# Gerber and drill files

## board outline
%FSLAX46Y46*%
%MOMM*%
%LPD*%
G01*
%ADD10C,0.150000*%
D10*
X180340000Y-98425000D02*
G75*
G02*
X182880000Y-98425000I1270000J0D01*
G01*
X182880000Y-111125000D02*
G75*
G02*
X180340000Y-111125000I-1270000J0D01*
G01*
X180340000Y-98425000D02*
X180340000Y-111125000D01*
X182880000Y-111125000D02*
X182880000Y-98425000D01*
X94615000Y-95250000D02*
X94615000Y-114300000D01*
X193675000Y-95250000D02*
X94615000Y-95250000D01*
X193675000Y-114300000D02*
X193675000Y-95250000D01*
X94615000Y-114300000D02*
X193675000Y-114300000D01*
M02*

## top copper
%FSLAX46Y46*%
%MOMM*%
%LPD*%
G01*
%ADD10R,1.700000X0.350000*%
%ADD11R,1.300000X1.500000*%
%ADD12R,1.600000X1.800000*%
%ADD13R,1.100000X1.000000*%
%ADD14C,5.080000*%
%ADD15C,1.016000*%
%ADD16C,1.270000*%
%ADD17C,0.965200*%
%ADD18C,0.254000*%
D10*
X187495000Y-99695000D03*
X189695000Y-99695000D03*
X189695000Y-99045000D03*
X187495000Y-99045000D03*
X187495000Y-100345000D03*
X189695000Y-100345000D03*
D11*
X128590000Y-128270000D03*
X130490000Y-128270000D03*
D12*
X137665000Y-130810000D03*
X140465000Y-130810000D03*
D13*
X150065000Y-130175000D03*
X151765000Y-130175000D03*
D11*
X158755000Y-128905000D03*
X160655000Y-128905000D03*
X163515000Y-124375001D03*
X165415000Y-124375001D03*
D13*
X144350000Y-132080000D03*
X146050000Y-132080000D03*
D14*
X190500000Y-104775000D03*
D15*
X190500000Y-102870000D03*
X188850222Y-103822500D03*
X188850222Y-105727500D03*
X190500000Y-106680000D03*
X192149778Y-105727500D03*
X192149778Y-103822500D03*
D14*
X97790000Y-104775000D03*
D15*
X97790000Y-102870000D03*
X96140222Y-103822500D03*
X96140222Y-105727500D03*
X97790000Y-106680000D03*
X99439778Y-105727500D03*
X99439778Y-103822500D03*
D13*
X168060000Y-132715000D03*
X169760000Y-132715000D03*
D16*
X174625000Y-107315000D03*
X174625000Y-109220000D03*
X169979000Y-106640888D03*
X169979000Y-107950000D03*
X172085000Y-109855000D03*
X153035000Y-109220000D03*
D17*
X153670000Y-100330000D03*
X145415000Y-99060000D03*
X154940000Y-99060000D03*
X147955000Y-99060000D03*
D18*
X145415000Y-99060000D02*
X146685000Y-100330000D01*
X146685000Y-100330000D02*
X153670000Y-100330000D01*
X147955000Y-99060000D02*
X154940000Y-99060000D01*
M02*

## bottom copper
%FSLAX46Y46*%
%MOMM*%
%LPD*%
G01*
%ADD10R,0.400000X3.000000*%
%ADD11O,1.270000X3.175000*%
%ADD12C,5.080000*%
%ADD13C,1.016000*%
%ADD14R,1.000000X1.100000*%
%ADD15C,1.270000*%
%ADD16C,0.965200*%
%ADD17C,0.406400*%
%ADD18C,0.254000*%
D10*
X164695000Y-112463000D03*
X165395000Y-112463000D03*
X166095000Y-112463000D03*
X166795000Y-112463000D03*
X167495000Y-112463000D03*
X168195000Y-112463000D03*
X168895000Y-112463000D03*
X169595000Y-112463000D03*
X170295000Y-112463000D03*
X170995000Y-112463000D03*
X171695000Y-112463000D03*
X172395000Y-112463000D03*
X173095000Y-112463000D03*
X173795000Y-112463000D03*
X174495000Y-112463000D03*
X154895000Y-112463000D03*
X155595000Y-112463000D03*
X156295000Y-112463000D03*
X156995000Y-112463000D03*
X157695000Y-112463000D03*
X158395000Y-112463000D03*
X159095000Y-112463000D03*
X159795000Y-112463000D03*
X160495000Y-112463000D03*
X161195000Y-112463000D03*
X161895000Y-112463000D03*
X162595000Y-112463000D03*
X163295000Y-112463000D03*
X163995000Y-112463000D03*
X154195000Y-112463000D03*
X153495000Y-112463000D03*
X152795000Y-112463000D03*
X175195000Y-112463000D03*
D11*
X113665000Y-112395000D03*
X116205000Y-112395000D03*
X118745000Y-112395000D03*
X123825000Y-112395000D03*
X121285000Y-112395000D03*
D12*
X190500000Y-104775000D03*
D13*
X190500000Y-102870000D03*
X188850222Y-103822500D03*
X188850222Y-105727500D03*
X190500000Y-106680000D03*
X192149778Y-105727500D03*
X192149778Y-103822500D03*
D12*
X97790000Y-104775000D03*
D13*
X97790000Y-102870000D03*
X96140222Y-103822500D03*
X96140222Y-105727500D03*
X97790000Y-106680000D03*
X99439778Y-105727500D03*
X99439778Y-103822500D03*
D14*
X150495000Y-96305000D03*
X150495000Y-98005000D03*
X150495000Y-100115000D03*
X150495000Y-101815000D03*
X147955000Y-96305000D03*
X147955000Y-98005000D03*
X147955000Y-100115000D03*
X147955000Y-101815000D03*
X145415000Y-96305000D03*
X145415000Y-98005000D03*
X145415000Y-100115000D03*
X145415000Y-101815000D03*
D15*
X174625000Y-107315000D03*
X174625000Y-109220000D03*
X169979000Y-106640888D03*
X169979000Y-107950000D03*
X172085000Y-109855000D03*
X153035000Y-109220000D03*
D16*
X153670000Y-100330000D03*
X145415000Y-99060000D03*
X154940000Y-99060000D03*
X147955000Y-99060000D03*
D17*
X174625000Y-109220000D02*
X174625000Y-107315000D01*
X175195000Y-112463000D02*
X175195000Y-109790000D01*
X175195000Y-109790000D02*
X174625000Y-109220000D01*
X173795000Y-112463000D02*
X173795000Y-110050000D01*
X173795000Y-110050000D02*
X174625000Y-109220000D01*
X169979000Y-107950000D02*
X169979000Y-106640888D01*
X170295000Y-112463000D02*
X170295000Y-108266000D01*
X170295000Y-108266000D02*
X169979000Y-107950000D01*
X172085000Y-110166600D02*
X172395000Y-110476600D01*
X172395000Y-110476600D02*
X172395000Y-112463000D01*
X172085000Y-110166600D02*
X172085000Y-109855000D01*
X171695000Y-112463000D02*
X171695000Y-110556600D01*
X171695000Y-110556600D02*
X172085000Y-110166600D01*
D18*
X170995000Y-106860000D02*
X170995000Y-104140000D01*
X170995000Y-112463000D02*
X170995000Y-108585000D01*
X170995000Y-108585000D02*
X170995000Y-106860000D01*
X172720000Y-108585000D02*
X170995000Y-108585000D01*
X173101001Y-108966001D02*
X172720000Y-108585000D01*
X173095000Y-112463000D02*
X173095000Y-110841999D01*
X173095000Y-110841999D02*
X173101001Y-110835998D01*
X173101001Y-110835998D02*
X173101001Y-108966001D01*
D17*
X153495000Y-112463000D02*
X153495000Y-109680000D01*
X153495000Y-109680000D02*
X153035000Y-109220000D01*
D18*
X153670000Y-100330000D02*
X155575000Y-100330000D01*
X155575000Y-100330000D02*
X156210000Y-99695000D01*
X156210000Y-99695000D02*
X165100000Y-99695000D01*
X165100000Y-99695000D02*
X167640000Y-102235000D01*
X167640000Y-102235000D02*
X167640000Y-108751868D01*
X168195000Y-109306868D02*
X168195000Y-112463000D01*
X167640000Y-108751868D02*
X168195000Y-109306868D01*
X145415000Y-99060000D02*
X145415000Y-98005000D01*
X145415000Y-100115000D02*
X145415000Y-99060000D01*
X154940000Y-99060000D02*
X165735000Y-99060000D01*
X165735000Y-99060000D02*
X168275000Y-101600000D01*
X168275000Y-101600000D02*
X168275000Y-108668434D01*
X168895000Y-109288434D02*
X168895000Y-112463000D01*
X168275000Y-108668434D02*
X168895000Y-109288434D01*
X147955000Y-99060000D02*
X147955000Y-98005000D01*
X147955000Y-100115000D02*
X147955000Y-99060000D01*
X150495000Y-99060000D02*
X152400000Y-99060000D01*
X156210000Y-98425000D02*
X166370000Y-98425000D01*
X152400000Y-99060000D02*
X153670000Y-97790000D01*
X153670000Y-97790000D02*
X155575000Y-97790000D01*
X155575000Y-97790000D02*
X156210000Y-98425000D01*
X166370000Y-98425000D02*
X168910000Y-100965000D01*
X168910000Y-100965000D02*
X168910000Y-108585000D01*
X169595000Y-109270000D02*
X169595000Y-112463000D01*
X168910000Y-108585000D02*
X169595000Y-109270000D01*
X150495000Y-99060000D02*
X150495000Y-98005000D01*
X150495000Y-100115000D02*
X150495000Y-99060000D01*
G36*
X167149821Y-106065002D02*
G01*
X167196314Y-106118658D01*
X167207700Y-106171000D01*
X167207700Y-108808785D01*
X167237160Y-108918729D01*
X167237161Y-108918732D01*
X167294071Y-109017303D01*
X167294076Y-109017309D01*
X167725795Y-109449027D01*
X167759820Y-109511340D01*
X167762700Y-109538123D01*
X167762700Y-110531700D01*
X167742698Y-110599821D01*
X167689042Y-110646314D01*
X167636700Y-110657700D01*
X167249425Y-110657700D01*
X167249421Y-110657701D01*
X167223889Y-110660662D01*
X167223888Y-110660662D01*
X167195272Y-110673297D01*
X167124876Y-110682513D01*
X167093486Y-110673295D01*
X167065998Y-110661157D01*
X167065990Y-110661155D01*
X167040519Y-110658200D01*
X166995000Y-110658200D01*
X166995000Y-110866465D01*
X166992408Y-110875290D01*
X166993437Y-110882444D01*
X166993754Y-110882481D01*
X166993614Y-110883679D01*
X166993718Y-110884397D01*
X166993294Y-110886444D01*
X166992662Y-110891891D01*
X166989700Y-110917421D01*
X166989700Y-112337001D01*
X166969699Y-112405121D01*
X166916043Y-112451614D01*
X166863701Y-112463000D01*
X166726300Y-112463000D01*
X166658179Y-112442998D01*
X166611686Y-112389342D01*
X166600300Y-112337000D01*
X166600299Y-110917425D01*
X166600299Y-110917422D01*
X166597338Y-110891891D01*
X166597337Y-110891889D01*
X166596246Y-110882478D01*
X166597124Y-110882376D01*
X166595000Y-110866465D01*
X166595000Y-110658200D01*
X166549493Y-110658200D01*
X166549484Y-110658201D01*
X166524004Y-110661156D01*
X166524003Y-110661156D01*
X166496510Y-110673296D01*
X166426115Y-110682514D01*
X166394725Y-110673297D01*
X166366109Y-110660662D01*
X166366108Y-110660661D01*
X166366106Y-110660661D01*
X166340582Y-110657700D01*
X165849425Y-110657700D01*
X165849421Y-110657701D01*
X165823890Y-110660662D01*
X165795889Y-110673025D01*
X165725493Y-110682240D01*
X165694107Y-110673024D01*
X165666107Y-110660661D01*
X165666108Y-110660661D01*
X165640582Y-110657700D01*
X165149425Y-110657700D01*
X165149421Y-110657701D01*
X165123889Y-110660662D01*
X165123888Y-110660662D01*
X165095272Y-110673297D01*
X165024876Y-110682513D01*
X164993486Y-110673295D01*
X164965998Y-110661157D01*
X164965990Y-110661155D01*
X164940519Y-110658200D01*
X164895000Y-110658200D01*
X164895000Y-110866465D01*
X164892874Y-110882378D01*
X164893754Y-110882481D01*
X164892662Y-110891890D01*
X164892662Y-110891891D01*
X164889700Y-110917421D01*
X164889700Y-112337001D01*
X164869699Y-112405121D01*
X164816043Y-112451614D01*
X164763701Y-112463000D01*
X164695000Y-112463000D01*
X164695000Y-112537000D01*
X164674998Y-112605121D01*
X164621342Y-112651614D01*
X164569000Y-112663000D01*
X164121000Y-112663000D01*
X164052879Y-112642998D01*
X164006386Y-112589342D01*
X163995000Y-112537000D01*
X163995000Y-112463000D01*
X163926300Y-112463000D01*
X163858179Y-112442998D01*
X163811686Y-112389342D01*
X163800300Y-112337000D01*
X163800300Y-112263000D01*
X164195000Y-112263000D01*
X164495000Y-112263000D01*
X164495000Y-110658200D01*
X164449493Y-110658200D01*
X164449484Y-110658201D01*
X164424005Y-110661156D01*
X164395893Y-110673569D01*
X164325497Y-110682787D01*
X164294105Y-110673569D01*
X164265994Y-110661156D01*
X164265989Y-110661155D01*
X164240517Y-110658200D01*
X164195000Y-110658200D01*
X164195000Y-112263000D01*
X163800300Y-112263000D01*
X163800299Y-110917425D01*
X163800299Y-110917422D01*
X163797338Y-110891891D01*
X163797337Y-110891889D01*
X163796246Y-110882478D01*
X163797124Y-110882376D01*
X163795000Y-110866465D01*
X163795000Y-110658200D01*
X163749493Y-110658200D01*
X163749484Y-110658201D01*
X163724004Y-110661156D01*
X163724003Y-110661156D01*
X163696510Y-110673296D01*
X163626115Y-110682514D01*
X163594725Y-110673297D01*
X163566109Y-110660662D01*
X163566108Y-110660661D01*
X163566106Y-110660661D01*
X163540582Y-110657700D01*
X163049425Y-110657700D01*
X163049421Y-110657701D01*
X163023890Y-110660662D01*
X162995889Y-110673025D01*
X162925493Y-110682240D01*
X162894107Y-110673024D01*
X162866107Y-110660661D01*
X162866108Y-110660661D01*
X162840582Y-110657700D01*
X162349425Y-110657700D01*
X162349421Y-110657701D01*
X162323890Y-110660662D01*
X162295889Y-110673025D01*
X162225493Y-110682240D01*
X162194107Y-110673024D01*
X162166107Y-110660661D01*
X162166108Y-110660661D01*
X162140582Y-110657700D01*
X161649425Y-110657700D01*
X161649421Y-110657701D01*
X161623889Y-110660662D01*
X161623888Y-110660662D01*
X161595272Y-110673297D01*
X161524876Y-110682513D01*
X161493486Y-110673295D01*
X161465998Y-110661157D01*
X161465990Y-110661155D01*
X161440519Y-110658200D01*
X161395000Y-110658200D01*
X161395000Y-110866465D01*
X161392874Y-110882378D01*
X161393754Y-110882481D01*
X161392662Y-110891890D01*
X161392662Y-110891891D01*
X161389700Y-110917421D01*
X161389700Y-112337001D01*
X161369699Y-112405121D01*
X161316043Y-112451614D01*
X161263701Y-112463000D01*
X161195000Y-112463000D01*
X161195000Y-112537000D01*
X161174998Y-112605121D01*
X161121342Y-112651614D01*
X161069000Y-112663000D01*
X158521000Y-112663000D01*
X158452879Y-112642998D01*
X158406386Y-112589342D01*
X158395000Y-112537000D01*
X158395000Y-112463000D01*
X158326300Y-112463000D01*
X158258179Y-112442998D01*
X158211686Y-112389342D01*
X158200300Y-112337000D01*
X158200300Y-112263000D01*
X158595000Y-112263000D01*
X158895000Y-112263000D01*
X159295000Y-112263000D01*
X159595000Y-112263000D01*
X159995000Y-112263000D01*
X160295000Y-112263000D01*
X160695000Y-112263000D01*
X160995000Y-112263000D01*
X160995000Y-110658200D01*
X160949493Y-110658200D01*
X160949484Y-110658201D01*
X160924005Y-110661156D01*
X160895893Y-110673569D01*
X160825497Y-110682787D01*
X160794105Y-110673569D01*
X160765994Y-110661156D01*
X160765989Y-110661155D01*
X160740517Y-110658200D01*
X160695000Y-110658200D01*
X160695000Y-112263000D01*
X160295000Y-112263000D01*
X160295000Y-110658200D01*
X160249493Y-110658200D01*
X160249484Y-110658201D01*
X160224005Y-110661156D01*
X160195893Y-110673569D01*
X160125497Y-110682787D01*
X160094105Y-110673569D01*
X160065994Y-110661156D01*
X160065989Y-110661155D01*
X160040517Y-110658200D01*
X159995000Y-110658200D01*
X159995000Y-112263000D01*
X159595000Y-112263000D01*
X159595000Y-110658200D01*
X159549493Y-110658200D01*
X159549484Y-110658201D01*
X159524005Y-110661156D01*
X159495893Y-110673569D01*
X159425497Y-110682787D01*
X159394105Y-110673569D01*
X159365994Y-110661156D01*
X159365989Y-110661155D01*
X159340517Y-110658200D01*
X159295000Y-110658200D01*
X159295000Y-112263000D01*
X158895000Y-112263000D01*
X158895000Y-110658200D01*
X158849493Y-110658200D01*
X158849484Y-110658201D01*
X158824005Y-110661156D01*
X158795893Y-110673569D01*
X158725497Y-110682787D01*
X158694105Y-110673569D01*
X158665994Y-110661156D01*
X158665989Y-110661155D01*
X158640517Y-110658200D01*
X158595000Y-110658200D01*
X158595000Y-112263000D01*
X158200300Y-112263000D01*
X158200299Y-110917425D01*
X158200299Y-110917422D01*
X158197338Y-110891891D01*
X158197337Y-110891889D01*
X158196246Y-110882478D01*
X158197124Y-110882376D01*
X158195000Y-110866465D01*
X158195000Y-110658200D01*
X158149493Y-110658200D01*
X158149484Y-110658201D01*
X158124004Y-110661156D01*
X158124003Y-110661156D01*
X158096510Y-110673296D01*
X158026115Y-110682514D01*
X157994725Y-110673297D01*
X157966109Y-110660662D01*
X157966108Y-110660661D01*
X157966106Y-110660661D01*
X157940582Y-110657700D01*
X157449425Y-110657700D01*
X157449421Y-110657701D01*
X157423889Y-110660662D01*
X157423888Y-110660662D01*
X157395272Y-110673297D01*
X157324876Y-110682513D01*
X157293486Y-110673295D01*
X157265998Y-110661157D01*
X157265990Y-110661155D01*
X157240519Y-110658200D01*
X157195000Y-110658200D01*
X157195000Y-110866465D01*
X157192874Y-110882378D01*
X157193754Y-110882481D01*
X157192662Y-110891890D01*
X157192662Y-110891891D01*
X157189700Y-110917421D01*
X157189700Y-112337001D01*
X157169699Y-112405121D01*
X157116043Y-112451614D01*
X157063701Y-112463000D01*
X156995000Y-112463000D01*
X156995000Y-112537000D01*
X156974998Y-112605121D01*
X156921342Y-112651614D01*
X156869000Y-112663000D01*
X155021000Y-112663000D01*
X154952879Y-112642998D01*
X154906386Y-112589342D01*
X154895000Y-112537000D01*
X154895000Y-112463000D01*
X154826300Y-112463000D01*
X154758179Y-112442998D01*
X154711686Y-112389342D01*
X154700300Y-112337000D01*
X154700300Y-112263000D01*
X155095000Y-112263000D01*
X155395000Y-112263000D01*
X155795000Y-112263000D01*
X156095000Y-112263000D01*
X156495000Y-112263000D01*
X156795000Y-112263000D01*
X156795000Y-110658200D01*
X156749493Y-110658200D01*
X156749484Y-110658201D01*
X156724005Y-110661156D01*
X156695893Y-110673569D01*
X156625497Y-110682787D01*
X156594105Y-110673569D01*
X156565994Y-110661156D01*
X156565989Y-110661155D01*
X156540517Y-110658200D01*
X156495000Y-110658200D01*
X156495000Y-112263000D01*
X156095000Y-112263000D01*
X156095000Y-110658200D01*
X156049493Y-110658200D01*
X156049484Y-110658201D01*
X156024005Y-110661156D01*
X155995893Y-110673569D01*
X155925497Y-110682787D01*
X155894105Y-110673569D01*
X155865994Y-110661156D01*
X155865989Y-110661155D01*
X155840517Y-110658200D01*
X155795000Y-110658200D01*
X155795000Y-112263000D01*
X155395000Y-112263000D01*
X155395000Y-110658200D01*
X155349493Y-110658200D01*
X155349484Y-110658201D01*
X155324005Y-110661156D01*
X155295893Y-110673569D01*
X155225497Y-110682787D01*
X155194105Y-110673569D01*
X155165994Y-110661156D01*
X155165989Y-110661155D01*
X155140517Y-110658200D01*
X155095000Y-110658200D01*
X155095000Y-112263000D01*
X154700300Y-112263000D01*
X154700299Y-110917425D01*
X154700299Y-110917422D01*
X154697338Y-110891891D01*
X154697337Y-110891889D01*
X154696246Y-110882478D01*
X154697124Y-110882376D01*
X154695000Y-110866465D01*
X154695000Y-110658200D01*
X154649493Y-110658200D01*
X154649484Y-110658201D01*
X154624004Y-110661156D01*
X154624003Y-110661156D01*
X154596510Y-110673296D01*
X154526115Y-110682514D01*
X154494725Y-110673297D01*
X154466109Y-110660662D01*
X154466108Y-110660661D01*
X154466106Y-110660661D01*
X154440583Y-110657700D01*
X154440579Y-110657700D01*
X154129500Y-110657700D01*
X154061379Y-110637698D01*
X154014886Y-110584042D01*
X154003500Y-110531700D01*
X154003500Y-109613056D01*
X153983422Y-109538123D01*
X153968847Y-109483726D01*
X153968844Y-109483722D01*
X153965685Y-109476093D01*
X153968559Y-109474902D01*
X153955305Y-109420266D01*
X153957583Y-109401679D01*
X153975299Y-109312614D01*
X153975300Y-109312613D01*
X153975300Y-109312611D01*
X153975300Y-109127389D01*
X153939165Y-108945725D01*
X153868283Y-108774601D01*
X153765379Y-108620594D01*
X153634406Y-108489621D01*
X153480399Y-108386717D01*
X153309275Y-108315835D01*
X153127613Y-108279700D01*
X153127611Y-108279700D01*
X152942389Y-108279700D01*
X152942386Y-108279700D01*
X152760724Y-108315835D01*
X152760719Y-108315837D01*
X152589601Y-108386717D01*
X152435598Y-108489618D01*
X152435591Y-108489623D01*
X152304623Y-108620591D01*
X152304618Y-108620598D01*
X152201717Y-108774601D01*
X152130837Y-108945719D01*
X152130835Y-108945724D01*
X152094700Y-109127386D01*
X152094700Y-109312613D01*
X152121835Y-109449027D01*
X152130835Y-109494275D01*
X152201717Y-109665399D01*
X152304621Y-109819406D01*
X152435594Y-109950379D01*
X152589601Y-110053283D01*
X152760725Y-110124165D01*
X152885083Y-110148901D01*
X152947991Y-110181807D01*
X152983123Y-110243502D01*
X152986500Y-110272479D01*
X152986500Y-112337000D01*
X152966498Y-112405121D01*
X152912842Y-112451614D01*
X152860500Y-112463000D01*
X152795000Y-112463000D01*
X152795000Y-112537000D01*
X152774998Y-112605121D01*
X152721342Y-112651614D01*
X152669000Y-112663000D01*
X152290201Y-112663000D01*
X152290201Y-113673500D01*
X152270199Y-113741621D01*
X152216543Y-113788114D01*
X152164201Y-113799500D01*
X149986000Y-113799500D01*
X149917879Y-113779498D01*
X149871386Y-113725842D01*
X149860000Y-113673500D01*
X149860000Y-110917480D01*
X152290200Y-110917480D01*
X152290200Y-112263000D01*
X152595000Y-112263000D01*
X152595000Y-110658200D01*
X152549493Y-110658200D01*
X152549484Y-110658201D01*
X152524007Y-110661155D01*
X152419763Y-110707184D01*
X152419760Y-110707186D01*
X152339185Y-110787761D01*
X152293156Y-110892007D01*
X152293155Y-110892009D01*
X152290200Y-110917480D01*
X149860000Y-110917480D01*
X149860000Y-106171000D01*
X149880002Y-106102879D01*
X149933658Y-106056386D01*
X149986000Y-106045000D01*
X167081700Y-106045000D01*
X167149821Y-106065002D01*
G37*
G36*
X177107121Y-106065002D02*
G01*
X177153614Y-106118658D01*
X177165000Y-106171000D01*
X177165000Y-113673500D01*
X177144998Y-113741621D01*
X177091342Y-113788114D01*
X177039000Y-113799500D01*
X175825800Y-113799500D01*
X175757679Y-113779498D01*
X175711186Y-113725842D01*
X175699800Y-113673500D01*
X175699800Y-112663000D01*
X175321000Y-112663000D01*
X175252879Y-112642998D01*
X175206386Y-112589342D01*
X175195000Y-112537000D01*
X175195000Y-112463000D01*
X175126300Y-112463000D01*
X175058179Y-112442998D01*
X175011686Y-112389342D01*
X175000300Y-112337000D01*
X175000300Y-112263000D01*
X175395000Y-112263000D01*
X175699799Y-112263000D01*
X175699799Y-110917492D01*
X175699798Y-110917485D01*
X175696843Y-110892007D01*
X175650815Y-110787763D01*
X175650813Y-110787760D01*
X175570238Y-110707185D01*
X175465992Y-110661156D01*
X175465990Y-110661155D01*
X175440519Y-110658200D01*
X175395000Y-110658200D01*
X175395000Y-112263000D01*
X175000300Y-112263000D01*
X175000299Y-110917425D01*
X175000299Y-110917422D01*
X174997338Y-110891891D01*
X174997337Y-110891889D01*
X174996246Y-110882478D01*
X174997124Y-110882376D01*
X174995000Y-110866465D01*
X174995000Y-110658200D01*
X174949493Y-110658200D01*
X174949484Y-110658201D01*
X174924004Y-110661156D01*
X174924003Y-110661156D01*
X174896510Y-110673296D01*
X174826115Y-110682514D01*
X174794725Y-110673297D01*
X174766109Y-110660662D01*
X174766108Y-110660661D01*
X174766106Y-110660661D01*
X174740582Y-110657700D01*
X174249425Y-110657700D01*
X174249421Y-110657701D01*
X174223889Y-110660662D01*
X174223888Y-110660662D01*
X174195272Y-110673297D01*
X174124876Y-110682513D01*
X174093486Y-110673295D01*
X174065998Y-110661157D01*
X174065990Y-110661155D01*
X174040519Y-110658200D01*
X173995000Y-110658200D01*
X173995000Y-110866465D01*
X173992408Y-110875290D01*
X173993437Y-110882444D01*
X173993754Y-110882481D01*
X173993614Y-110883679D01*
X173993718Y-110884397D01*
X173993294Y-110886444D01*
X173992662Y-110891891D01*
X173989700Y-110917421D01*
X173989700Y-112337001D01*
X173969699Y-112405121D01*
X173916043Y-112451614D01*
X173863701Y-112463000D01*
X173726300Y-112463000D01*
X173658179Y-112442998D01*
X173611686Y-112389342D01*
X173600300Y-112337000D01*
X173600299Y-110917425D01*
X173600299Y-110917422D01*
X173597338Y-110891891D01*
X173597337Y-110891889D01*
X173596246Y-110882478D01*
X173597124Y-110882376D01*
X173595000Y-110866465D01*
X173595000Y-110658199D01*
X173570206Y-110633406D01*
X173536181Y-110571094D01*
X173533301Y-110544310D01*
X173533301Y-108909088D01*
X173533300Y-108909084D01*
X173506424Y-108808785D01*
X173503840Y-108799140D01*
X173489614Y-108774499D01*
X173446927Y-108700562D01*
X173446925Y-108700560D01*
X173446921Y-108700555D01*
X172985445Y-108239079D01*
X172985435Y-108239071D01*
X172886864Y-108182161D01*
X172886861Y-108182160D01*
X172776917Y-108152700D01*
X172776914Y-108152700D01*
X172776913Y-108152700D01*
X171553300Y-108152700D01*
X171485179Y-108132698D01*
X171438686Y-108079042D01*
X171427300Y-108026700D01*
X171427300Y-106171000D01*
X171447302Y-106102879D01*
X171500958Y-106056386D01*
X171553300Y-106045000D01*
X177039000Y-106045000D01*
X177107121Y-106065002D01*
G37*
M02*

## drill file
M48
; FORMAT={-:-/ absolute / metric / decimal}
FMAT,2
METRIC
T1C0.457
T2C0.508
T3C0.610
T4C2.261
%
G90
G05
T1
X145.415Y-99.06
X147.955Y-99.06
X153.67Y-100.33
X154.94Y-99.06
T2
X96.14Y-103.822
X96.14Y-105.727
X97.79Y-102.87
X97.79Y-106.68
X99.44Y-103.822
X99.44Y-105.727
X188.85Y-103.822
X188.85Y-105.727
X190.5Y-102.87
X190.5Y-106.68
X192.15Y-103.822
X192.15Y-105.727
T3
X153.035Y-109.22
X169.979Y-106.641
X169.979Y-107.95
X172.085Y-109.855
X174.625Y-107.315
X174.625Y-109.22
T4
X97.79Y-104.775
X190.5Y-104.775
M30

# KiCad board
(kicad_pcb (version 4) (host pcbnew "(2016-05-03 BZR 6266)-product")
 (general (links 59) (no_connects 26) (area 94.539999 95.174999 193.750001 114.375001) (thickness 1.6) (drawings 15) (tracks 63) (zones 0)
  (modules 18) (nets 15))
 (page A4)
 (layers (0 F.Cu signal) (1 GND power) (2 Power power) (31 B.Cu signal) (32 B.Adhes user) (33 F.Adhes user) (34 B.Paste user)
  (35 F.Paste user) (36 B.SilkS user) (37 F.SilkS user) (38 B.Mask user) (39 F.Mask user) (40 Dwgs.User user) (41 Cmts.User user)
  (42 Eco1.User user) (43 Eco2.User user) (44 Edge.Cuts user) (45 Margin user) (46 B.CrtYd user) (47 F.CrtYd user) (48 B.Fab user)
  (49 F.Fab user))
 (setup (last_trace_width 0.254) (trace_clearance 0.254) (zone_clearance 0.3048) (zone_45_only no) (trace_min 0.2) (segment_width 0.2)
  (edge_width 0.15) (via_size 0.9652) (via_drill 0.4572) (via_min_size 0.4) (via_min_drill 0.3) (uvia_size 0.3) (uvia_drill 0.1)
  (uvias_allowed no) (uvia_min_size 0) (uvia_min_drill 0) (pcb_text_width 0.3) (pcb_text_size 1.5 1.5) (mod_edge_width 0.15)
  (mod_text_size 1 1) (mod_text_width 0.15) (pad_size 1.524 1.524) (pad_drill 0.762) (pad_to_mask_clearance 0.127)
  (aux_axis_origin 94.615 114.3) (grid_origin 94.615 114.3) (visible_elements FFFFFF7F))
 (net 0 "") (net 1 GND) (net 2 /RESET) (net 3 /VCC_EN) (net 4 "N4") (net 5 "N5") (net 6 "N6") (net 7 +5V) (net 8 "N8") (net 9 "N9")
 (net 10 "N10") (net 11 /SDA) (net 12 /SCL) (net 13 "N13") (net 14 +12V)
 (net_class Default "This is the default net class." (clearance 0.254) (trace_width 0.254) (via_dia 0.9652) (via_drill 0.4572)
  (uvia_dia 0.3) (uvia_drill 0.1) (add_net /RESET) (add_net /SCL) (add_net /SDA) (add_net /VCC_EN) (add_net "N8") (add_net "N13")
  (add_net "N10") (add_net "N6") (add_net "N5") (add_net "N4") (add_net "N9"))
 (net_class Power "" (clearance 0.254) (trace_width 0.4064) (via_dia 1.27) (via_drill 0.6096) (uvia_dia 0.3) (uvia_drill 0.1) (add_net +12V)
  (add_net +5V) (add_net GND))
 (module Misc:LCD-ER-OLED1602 (layer F.Cu) (at 144.145 104.013)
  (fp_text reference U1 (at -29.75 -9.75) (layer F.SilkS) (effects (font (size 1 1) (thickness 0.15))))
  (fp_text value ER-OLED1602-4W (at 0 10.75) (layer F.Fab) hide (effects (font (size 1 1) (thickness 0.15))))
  (pad 16 smd rect (at 20.55 8.45) (size 0.4 3) (layers B.Cu B.Paste B.Mask) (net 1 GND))
  (pad 15 smd rect (at 21.25 8.45) (size 0.4 3) (layers B.Cu B.Paste B.Mask))
  (pad 14 smd rect (at 21.95 8.45) (size 0.4 3) (layers B.Cu B.Paste B.Mask) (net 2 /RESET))
  (pad 13 smd rect (at 22.65 8.45) (size 0.4 3) (layers B.Cu B.Paste B.Mask) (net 1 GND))
  (pad 12 smd rect (at 23.35 8.45) (size 0.4 3) (layers B.Cu B.Paste B.Mask) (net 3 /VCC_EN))
  (pad 11 smd rect (at 24.05 8.45) (size 0.4 3) (layers B.Cu B.Paste B.Mask) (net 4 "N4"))
  (pad 10 smd rect (at 24.75 8.45) (size 0.4 3) (layers B.Cu B.Paste B.Mask) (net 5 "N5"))
  (pad 9 smd rect (at 25.45 8.45) (size 0.4 3) (layers B.Cu B.Paste B.Mask) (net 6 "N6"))
  (pad 8 smd rect (at 26.15 8.45) (size 0.4 3) (layers B.Cu B.Paste B.Mask) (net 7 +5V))
  (pad 7 smd rect (at 26.85 8.45) (size 0.4 3) (layers B.Cu B.Paste B.Mask) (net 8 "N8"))
  (pad 6 smd rect (at 27.55 8.45) (size 0.4 3) (layers B.Cu B.Paste B.Mask) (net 7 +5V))
  (pad 5 smd rect (at 28.25 8.45) (size 0.4 3) (layers B.Cu B.Paste B.Mask) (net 7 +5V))
  (pad 4 smd rect (at 28.95 8.45) (size 0.4 3) (layers B.Cu B.Paste B.Mask) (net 8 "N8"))
  (pad 3 smd rect (at 29.65 8.45) (size 0.4 3) (layers B.Cu B.Paste B.Mask) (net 1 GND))
  (pad 2 smd rect (at 30.35 8.45) (size 0.4 3) (layers B.Cu B.Paste B.Mask) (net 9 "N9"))
  (pad 30 smd rect (at 10.75 8.45) (size 0.4 3) (layers B.Cu B.Paste B.Mask) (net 1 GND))
  (pad 29 smd rect (at 11.45 8.45) (size 0.4 3) (layers B.Cu B.Paste B.Mask) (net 1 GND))
  (pad 28 smd rect (at 12.15 8.45) (size 0.4 3) (layers B.Cu B.Paste B.Mask) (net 1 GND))
  (pad 27 smd rect (at 12.85 8.45) (size 0.4 3) (layers B.Cu B.Paste B.Mask) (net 1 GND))
  (pad 26 smd rect (at 13.55 8.45) (size 0.4 3) (layers B.Cu B.Paste B.Mask) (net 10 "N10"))
  (pad 25 smd rect (at 14.25 8.45) (size 0.4 3) (layers B.Cu B.Paste B.Mask) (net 1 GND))
  (pad 24 smd rect (at 14.95 8.45) (size 0.4 3) (layers B.Cu B.Paste B.Mask) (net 1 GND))
  (pad 23 smd rect (at 15.65 8.45) (size 0.4 3) (layers B.Cu B.Paste B.Mask) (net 1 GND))
  (pad 22 smd rect (at 16.35 8.45) (size 0.4 3) (layers B.Cu B.Paste B.Mask) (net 1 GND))
  (pad 21 smd rect (at 17.05 8.45) (size 0.4 3) (layers B.Cu B.Paste B.Mask) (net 1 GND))
  (pad 20 smd rect (at 17.75 8.45) (size 0.4 3) (layers B.Cu B.Paste B.Mask) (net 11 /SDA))
  (pad 19 smd rect (at 18.45 8.45) (size 0.4 3) (layers B.Cu B.Paste B.Mask) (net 11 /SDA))
  (pad 18 smd rect (at 19.15 8.45) (size 0.4 3) (layers B.Cu B.Paste B.Mask) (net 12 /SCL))
  (pad 17 smd rect (at 19.85 8.45) (size 0.4 3) (layers B.Cu B.Paste B.Mask) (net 1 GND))
  (pad 31 smd rect (at 10.05 8.45) (size 0.4 3) (layers B.Cu B.Paste B.Mask) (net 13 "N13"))
  (pad 32 smd rect (at 9.35 8.45) (size 0.4 3) (layers B.Cu B.Paste B.Mask) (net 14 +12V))
  (pad 33 smd rect (at 8.65 8.45) (size 0.4 3) (layers B.Cu B.Paste B.Mask) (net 1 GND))
  (pad 1 smd rect (at 31.05 8.45) (size 0.4 3) (layers B.Cu B.Paste B.Mask) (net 1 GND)))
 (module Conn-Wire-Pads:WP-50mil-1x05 (layer B.Cu) (at 118.745 112.395)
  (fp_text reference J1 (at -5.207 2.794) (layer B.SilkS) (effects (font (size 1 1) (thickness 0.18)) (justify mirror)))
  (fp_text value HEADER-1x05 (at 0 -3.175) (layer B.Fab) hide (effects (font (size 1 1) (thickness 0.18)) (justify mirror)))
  (pad 1 smd oval (at -5.08 0) (size 1.27 3.175) (layers B.Cu B.Paste B.Mask) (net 7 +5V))
  (pad 2 smd oval (at -2.54 0) (size 1.27 3.175) (layers B.Cu B.Paste B.Mask) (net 11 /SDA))
  (pad 3 smd oval (at 0 0) (size 1.27 3.175) (layers B.Cu B.Paste B.Mask) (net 12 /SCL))
  (pad 5 smd oval (at 5.08 0) (size 1.27 3.175) (layers B.Cu B.Paste B.Mask) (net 1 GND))
  (pad 4 smd oval (at 2.54 0) (size 1.27 3.175) (layers B.Cu B.Paste B.Mask) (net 2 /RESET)))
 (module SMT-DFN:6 (layer F.Cu) (at 188.595 99.695)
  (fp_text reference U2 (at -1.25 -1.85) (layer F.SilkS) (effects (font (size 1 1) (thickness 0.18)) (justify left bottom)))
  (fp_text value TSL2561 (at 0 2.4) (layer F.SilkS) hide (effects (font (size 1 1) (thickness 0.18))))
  (pad 2 smd rect (at -1.1 0) (size 1.7 0.35) (layers F.Cu F.Paste F.Mask))
  (pad 5 smd rect (at 1.1 0) (size 1.7 0.35) (layers F.Cu F.Paste F.Mask))
  (pad 6 smd rect (at 1.1 -0.65) (size 1.7 0.35) (layers F.Cu F.Paste F.Mask))
  (pad 1 smd rect (at -1.1 -0.65) (size 1.7 0.35) (layers F.Cu F.Paste F.Mask))
  (pad 3 smd rect (at -1.1 0.65) (size 1.7 0.35) (layers F.Cu F.Paste F.Mask))
  (pad 4 smd rect (at 1.1 0.65) (size 1.7 0.35) (layers F.Cu F.Paste F.Mask)))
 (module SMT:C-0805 (layer F.Cu) (at 129.54 128.27)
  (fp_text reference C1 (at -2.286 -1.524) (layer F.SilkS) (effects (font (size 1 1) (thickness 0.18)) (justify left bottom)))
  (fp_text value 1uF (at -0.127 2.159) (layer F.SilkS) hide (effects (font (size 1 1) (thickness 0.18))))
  (pad 1 smd rect (at -0.95 0) (size 1.3 1.5) (layers F.Cu F.Paste F.Mask) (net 1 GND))
  (pad 2 smd rect (at 0.95 0) (size 1.3 1.5) (layers F.Cu F.Paste F.Mask) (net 8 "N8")))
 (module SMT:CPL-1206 (layer F.Cu) (at 139.065 130.81)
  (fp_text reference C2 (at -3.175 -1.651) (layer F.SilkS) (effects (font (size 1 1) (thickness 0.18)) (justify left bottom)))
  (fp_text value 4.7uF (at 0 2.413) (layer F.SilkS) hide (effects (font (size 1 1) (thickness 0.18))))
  (pad A smd rect (at -1.4 0) (size 1.6 1.8) (layers F.Cu F.Paste F.Mask) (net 13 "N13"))
  (pad K smd rect (at 1.4 0) (size 1.6 1.8) (layers F.Cu F.Paste F.Mask) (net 1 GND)))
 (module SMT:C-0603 (layer F.Cu) (at 150.915 130.175)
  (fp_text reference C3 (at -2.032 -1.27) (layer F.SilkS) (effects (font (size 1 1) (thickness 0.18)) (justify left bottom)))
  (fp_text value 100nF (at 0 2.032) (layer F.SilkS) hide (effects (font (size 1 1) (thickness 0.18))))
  (pad 1 smd rect (at -0.85 0) (size 1.1 1) (layers F.Cu F.Paste F.Mask) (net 1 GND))
  (pad 2 smd rect (at 0.85 0) (size 1.1 1) (layers F.Cu F.Paste F.Mask) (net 7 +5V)))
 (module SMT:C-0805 (layer F.Cu) (at 159.705 128.905)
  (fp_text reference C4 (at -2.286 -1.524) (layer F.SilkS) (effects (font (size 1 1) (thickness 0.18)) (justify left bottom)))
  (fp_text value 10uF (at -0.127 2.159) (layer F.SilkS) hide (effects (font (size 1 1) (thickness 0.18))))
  (pad 1 smd rect (at -0.95 0) (size 1.3 1.5) (layers F.Cu F.Paste F.Mask))
  (pad 2 smd rect (at 0.95 0) (size 1.3 1.5) (layers F.Cu F.Paste F.Mask)))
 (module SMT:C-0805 (layer F.Cu) (at 164.465 124.375001)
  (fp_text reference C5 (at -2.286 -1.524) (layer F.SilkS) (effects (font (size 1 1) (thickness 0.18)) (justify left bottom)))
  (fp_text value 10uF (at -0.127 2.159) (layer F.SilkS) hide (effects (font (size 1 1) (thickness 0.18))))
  (pad 1 smd rect (at -0.95 0) (size 1.3 1.5) (layers F.Cu F.Paste F.Mask))
  (pad 2 smd rect (at 0.95 0) (size 1.3 1.5) (layers F.Cu F.Paste F.Mask)))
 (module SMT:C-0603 (layer F.Cu) (at 145.2 132.08)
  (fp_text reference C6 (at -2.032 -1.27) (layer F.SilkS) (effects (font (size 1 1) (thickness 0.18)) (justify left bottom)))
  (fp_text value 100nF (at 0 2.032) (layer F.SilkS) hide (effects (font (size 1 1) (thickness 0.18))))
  (pad 1 smd rect (at -0.85 0) (size 1.1 1) (layers F.Cu F.Paste F.Mask) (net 1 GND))
  (pad 2 smd rect (at 0.85 0) (size 1.1 1) (layers F.Cu F.Paste F.Mask) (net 14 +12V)))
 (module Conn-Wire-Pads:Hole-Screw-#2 (layer F.Cu) (at 190.5 104.775)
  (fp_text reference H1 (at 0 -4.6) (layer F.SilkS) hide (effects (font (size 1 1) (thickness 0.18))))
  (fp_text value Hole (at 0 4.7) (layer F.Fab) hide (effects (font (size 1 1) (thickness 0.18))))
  (pad P thru_hole circle (at 0 0) (size 5.08 5.08) (drill 2.2606) (layers *.Cu *.Mask) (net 1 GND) (clearance 1.016) (zone_connect 2))
  (pad P thru_hole circle (at 0 -1.905) (size 1.016 1.016) (drill 0.508) (layers *.Cu) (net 1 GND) (clearance 0.0254) (zone_connect 2))
  (pad P thru_hole circle (at -1.649778 -0.9525 60) (size 1.016 1.016) (drill 0.508) (layers *.Cu) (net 1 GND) (clearance 0.0254)
   (zone_connect 2))
  (pad P thru_hole circle (at -1.649778 0.9525 120) (size 1.016 1.016) (drill 0.508) (layers *.Cu) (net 1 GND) (clearance 0.0254)
   (zone_connect 2))
  (pad P thru_hole circle (at 0 1.905 180) (size 1.016 1.016) (drill 0.508) (layers *.Cu) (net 1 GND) (clearance 0.0254) (zone_connect 2))
  (pad P thru_hole circle (at 1.649778 0.9525 240) (size 1.016 1.016) (drill 0.508) (layers *.Cu) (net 1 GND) (clearance 0.0254)
   (zone_connect 2))
  (pad P thru_hole circle (at 1.649778 -0.9525 300) (size 1.016 1.016) (drill 0.508) (layers *.Cu) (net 1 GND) (clearance 0.0254)
   (zone_connect 2)))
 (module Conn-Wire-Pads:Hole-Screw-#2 (layer F.Cu) (at 97.79 104.775)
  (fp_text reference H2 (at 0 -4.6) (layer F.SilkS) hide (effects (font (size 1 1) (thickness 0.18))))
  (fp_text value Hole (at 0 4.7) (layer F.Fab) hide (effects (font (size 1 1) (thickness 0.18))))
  (pad P thru_hole circle (at 0 0) (size 5.08 5.08) (drill 2.2606) (layers *.Cu *.Mask) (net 1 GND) (clearance 1.016) (zone_connect 2))
  (pad P thru_hole circle (at 0 -1.905) (size 1.016 1.016) (drill 0.508) (layers *.Cu) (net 1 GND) (clearance 0.0254) (zone_connect 2))
  (pad P thru_hole circle (at -1.649778 -0.9525 60) (size 1.016 1.016) (drill 0.508) (layers *.Cu) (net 1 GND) (clearance 0.0254)
   (zone_connect 2))
  (pad P thru_hole circle (at -1.649778 0.9525 120) (size 1.016 1.016) (drill 0.508) (layers *.Cu) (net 1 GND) (clearance 0.0254)
   (zone_connect 2))
  (pad P thru_hole circle (at 0 1.905 180) (size 1.016 1.016) (drill 0.508) (layers *.Cu) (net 1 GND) (clearance 0.0254) (zone_connect 2))
  (pad P thru_hole circle (at 1.649778 0.9525 240) (size 1.016 1.016) (drill 0.508) (layers *.Cu) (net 1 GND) (clearance 0.0254)
   (zone_connect 2))
  (pad P thru_hole circle (at 1.649778 -0.9525 300) (size 1.016 1.016) (drill 0.508) (layers *.Cu) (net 1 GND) (clearance 0.0254)
   (zone_connect 2)))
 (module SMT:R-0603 (layer F.Cu) (at 168.91 132.715)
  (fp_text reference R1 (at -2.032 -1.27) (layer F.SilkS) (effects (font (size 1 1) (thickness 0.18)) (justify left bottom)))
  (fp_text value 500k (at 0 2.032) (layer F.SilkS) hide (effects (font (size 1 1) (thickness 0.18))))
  (pad 1 smd rect (at -0.85 0) (size 1.1 1) (layers F.Cu F.Paste F.Mask) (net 10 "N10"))
  (pad 2 smd rect (at 0.85 0) (size 1.1 1) (layers F.Cu F.Paste F.Mask) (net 1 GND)))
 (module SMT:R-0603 (layer B.Cu) (at 150.495 97.155 270)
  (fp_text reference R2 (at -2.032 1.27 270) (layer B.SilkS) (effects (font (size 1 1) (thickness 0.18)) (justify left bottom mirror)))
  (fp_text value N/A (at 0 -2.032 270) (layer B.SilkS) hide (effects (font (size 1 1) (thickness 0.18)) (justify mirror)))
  (pad 1 smd rect (at -0.85 0 270) (size 1.1 1) (layers B.Cu B.Paste B.Mask) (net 7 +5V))
  (pad 2 smd rect (at 0.85 0 270) (size 1.1 1) (layers B.Cu B.Paste B.Mask) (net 6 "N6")))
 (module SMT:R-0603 (layer B.Cu) (at 150.495 100.965 270)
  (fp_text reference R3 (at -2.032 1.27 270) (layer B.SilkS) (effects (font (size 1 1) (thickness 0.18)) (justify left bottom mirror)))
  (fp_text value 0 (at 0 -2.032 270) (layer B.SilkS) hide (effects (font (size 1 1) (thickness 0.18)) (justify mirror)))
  (pad 1 smd rect (at -0.85 0 270) (size 1.1 1) (layers B.Cu B.Paste B.Mask) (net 6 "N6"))
  (pad 2 smd rect (at 0.85 0 270) (size 1.1 1) (layers B.Cu B.Paste B.Mask) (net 1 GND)))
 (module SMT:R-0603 (layer B.Cu) (at 147.955 97.155 270)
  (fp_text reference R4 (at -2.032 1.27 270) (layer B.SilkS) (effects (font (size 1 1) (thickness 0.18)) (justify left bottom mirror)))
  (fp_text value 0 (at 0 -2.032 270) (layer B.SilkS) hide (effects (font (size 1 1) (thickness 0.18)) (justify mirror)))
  (pad 1 smd rect (at -0.85 0 270) (size 1.1 1) (layers B.Cu B.Paste B.Mask) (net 7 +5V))
  (pad 2 smd rect (at 0.85 0 270) (size 1.1 1) (layers B.Cu B.Paste B.Mask) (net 5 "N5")))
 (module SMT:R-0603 (layer B.Cu) (at 147.955 100.965 270)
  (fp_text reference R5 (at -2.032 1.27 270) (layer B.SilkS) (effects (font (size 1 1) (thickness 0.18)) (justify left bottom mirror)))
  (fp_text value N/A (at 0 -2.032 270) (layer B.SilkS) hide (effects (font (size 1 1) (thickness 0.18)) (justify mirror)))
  (pad 1 smd rect (at -0.85 0 270) (size 1.1 1) (layers B.Cu B.Paste B.Mask) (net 5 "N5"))
  (pad 2 smd rect (at 0.85 0 270) (size 1.1 1) (layers B.Cu B.Paste B.Mask) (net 1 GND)))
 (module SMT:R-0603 (layer B.Cu) (at 145.415 97.155 270)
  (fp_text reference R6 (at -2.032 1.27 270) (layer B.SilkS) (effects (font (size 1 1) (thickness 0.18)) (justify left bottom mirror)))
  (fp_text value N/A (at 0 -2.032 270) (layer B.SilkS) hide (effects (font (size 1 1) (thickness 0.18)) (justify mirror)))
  (pad 1 smd rect (at -0.85 0 270) (size 1.1 1) (layers B.Cu B.Paste B.Mask) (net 7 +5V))
  (pad 2 smd rect (at 0.85 0 270) (size 1.1 1) (layers B.Cu B.Paste B.Mask) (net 4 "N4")))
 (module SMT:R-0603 (layer B.Cu) (at 145.415 100.965 270)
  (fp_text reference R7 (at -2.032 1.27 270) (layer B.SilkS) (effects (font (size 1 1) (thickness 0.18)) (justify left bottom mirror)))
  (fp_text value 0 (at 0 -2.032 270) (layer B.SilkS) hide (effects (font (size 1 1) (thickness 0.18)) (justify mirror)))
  (pad 1 smd rect (at -0.85 0 270) (size 1.1 1) (layers B.Cu B.Paste B.Mask) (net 4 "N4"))
  (pad 2 smd rect (at 0.85 0 270) (size 1.1 1) (layers B.Cu B.Paste B.Mask) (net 1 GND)))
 (gr_arc (start 181.61 98.425) (end 180.34 98.425) (angle 180) (layer Edge.Cuts) (width 0.15))
 (gr_arc (start 181.61 111.125) (end 182.88 111.125) (angle 180) (layer Edge.Cuts) (width 0.15))
 (gr_line (start 180.34 98.425) (end 180.34 111.125) (layer Edge.Cuts) (width 0.15))
 (gr_line (start 182.88 111.125) (end 182.88 98.425) (layer Edge.Cuts) (width 0.15))
 (gr_line (start 94.615 95.25) (end 94.615 114.3) (angle 90) (layer Edge.Cuts) (width 0.15))
 (gr_line (start 193.675 95.25) (end 94.615 95.25) (angle 90) (layer Edge.Cuts) (width 0.15))
 (gr_line (start 193.675 114.3) (end 193.675 95.25) (angle 90) (layer Edge.Cuts) (width 0.15))
 (gr_line (start 94.615 114.3) (end 193.675 114.3) (angle 90) (layer Edge.Cuts) (width 0.15))
 (segment (start 174.625 109.22) (end 174.625 107.315) (width 0.4064) (layer B.Cu) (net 1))
 (via (at 174.625 107.315) (size 1.27) (drill 0.6096) (layers F.Cu B.Cu) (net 1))
 (segment (start 175.195 112.463) (end 175.195 109.79) (width 0.4064) (layer B.Cu) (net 1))
 (segment (start 175.195 109.79) (end 174.625 109.22) (width 0.4064) (layer B.Cu) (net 1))
 (segment (start 173.795 112.463) (end 173.795 110.05) (width 0.4064) (layer B.Cu) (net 1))
 (segment (start 173.795 110.05) (end 174.625 109.22) (width 0.4064) (layer B.Cu) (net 1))
 (via (at 174.625 109.22) (size 1.27) (drill 0.6096) (layers F.Cu B.Cu) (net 1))
 (segment (start 169.979 107.95) (end 169.979 106.640888) (width 0.4064) (layer B.Cu) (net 7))
 (via (at 169.979 106.640888) (size 1.27) (drill 0.6096) (layers F.Cu B.Cu) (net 7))
 (segment (start 170.295 112.463) (end 170.295 108.266) (width 0.4064) (layer B.Cu) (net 7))
 (segment (start 170.295 108.266) (end 169.979 107.95) (width 0.4064) (layer B.Cu) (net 7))
 (via (at 169.979 107.95) (size 1.27) (drill 0.6096) (layers F.Cu B.Cu) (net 7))
 (via (at 172.085 109.855) (size 1.27) (drill 0.6096) (layers F.Cu B.Cu) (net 7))
 (segment (start 172.085 110.1666) (end 172.395 110.4766) (width 0.4064) (layer B.Cu) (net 7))
 (segment (start 172.395 110.4766) (end 172.395 112.463) (width 0.4064) (layer B.Cu) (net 7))
 (segment (start 172.085 110.1666) (end 172.085 109.855) (width 0.4064) (layer B.Cu) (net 7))
 (segment (start 171.695 112.463) (end 171.695 110.5566) (width 0.4064) (layer B.Cu) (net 7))
 (segment (start 171.695 110.5566) (end 172.085 110.1666) (width 0.4064) (layer B.Cu) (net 7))
 (segment (start 170.995 106.86) (end 170.995 104.14) (width 0.254) (layer B.Cu) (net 8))
 (segment (start 170.995 112.463) (end 170.995 108.585) (width 0.254) (layer B.Cu) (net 8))
 (segment (start 170.995 108.585) (end 170.995 106.86) (width 0.254) (layer B.Cu) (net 8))
 (segment (start 172.72 108.585) (end 170.995 108.585) (width 0.254) (layer B.Cu) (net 8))
 (segment (start 173.101001 108.966001) (end 172.72 108.585) (width 0.254) (layer B.Cu) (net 8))
 (segment (start 173.095 112.463) (end 173.095 110.841999) (width 0.254) (layer B.Cu) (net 8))
 (segment (start 173.095 110.841999) (end 173.101001 110.835998) (width 0.254) (layer B.Cu) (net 8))
 (segment (start 173.101001 110.835998) (end 173.101001 108.966001) (width 0.254) (layer B.Cu) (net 8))
 (segment (start 153.495 112.463) (end 153.495 109.68) (width 0.4064) (layer B.Cu) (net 14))
 (segment (start 153.495 109.68) (end 153.035 109.22) (width 0.4064) (layer B.Cu) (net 14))
 (via (at 153.035 109.22) (size 1.27) (drill 0.6096) (layers F.Cu B.Cu) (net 14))
 (segment (start 153.67 100.33) (end 155.575 100.33) (width 0.254) (layer B.Cu) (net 4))
 (segment (start 155.575 100.33) (end 156.21 99.695) (width 0.254) (layer B.Cu) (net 4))
 (segment (start 156.21 99.695) (end 165.1 99.695) (width 0.254) (layer B.Cu) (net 4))
 (segment (start 165.1 99.695) (end 167.64 102.235) (width 0.254) (layer B.Cu) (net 4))
 (segment (start 167.64 102.235) (end 167.64 108.751868) (width 0.254) (layer B.Cu) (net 4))
 (segment (start 168.195 109.306868) (end 168.195 112.463) (width 0.254) (layer B.Cu) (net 4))
 (segment (start 167.64 108.751868) (end 168.195 109.306868) (width 0.254) (layer B.Cu) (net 4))
 (via (at 153.67 100.33) (size 0.9652) (drill 0.4572) (layers F.Cu B.Cu) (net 4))
 (segment (start 145.415 99.06) (end 146.685 100.33) (width 0.254) (layer F.Cu) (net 4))
 (segment (start 146.685 100.33) (end 153.67 100.33) (width 0.254) (layer F.Cu) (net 4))
 (segment (start 145.415 99.06) (end 145.415 98.005) (width 0.254) (layer B.Cu) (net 4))
 (segment (start 145.415 100.115) (end 145.415 99.06) (width 0.254) (layer B.Cu) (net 4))
 (via (at 145.415 99.06) (size 0.9652) (drill 0.4572) (layers F.Cu B.Cu) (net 4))
 (segment (start 154.94 99.06) (end 165.735 99.06) (width 0.254) (layer B.Cu) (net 5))
 (segment (start 165.735 99.06) (end 168.275 101.6) (width 0.254) (layer B.Cu) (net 5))
 (segment (start 168.275 101.6) (end 168.275 108.668434) (width 0.254) (layer B.Cu) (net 5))
 (segment (start 168.895 109.288434) (end 168.895 112.463) (width 0.254) (layer B.Cu) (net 5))
 (segment (start 168.275 108.668434) (end 168.895 109.288434) (width 0.254) (layer B.Cu) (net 5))
 (via (at 154.94 99.06) (size 0.9652) (drill 0.4572) (layers F.Cu B.Cu) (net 5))
 (segment (start 147.955 99.06) (end 154.94 99.06) (width 0.254) (layer F.Cu) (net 5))
 (segment (start 147.955 99.06) (end 147.955 98.005) (width 0.254) (layer B.Cu) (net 5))
 (segment (start 147.955 100.115) (end 147.955 99.06) (width 0.254) (layer B.Cu) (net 5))
 (via (at 147.955 99.06) (size 0.9652) (drill 0.4572) (layers F.Cu B.Cu) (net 5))
 (segment (start 150.495 99.06) (end 152.4 99.06) (width 0.254) (layer B.Cu) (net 6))
 (segment (start 156.21 98.425) (end 166.37 98.425) (width 0.254) (layer B.Cu) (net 6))
 (segment (start 152.4 99.06) (end 153.67 97.79) (width 0.254) (layer B.Cu) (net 6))
 (segment (start 153.67 97.79) (end 155.575 97.79) (width 0.254) (layer B.Cu) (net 6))
 (segment (start 155.575 97.79) (end 156.21 98.425) (width 0.254) (layer B.Cu) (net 6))
 (segment (start 166.37 98.425) (end 168.91 100.965) (width 0.254) (layer B.Cu) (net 6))
 (segment (start 168.91 100.965) (end 168.91 108.585) (width 0.254) (layer B.Cu) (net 6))
 (segment (start 169.595 109.27) (end 169.595 112.463) (width 0.254) (layer B.Cu) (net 6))
 (segment (start 168.91 108.585) (end 169.595 109.27) (width 0.254) (layer B.Cu) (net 6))
 (segment (start 150.495 99.06) (end 150.495 98.005) (width 0.254) (layer B.Cu) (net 6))
 (segment (start 150.495 100.115) (end 150.495 99.06) (width 0.254) (layer B.Cu) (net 6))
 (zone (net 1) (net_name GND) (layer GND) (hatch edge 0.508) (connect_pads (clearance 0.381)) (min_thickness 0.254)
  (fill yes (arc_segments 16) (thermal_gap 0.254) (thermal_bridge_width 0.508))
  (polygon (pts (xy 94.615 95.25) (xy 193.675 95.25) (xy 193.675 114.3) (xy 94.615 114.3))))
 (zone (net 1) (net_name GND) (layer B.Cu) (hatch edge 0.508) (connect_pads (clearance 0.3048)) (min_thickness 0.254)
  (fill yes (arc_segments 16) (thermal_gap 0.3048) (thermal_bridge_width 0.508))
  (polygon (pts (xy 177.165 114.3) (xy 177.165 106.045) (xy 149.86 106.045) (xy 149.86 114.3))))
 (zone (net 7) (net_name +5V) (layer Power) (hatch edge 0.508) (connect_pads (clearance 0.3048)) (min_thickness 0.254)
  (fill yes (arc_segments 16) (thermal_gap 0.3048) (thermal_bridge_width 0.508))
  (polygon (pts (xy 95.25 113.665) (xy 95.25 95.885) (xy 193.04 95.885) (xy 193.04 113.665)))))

